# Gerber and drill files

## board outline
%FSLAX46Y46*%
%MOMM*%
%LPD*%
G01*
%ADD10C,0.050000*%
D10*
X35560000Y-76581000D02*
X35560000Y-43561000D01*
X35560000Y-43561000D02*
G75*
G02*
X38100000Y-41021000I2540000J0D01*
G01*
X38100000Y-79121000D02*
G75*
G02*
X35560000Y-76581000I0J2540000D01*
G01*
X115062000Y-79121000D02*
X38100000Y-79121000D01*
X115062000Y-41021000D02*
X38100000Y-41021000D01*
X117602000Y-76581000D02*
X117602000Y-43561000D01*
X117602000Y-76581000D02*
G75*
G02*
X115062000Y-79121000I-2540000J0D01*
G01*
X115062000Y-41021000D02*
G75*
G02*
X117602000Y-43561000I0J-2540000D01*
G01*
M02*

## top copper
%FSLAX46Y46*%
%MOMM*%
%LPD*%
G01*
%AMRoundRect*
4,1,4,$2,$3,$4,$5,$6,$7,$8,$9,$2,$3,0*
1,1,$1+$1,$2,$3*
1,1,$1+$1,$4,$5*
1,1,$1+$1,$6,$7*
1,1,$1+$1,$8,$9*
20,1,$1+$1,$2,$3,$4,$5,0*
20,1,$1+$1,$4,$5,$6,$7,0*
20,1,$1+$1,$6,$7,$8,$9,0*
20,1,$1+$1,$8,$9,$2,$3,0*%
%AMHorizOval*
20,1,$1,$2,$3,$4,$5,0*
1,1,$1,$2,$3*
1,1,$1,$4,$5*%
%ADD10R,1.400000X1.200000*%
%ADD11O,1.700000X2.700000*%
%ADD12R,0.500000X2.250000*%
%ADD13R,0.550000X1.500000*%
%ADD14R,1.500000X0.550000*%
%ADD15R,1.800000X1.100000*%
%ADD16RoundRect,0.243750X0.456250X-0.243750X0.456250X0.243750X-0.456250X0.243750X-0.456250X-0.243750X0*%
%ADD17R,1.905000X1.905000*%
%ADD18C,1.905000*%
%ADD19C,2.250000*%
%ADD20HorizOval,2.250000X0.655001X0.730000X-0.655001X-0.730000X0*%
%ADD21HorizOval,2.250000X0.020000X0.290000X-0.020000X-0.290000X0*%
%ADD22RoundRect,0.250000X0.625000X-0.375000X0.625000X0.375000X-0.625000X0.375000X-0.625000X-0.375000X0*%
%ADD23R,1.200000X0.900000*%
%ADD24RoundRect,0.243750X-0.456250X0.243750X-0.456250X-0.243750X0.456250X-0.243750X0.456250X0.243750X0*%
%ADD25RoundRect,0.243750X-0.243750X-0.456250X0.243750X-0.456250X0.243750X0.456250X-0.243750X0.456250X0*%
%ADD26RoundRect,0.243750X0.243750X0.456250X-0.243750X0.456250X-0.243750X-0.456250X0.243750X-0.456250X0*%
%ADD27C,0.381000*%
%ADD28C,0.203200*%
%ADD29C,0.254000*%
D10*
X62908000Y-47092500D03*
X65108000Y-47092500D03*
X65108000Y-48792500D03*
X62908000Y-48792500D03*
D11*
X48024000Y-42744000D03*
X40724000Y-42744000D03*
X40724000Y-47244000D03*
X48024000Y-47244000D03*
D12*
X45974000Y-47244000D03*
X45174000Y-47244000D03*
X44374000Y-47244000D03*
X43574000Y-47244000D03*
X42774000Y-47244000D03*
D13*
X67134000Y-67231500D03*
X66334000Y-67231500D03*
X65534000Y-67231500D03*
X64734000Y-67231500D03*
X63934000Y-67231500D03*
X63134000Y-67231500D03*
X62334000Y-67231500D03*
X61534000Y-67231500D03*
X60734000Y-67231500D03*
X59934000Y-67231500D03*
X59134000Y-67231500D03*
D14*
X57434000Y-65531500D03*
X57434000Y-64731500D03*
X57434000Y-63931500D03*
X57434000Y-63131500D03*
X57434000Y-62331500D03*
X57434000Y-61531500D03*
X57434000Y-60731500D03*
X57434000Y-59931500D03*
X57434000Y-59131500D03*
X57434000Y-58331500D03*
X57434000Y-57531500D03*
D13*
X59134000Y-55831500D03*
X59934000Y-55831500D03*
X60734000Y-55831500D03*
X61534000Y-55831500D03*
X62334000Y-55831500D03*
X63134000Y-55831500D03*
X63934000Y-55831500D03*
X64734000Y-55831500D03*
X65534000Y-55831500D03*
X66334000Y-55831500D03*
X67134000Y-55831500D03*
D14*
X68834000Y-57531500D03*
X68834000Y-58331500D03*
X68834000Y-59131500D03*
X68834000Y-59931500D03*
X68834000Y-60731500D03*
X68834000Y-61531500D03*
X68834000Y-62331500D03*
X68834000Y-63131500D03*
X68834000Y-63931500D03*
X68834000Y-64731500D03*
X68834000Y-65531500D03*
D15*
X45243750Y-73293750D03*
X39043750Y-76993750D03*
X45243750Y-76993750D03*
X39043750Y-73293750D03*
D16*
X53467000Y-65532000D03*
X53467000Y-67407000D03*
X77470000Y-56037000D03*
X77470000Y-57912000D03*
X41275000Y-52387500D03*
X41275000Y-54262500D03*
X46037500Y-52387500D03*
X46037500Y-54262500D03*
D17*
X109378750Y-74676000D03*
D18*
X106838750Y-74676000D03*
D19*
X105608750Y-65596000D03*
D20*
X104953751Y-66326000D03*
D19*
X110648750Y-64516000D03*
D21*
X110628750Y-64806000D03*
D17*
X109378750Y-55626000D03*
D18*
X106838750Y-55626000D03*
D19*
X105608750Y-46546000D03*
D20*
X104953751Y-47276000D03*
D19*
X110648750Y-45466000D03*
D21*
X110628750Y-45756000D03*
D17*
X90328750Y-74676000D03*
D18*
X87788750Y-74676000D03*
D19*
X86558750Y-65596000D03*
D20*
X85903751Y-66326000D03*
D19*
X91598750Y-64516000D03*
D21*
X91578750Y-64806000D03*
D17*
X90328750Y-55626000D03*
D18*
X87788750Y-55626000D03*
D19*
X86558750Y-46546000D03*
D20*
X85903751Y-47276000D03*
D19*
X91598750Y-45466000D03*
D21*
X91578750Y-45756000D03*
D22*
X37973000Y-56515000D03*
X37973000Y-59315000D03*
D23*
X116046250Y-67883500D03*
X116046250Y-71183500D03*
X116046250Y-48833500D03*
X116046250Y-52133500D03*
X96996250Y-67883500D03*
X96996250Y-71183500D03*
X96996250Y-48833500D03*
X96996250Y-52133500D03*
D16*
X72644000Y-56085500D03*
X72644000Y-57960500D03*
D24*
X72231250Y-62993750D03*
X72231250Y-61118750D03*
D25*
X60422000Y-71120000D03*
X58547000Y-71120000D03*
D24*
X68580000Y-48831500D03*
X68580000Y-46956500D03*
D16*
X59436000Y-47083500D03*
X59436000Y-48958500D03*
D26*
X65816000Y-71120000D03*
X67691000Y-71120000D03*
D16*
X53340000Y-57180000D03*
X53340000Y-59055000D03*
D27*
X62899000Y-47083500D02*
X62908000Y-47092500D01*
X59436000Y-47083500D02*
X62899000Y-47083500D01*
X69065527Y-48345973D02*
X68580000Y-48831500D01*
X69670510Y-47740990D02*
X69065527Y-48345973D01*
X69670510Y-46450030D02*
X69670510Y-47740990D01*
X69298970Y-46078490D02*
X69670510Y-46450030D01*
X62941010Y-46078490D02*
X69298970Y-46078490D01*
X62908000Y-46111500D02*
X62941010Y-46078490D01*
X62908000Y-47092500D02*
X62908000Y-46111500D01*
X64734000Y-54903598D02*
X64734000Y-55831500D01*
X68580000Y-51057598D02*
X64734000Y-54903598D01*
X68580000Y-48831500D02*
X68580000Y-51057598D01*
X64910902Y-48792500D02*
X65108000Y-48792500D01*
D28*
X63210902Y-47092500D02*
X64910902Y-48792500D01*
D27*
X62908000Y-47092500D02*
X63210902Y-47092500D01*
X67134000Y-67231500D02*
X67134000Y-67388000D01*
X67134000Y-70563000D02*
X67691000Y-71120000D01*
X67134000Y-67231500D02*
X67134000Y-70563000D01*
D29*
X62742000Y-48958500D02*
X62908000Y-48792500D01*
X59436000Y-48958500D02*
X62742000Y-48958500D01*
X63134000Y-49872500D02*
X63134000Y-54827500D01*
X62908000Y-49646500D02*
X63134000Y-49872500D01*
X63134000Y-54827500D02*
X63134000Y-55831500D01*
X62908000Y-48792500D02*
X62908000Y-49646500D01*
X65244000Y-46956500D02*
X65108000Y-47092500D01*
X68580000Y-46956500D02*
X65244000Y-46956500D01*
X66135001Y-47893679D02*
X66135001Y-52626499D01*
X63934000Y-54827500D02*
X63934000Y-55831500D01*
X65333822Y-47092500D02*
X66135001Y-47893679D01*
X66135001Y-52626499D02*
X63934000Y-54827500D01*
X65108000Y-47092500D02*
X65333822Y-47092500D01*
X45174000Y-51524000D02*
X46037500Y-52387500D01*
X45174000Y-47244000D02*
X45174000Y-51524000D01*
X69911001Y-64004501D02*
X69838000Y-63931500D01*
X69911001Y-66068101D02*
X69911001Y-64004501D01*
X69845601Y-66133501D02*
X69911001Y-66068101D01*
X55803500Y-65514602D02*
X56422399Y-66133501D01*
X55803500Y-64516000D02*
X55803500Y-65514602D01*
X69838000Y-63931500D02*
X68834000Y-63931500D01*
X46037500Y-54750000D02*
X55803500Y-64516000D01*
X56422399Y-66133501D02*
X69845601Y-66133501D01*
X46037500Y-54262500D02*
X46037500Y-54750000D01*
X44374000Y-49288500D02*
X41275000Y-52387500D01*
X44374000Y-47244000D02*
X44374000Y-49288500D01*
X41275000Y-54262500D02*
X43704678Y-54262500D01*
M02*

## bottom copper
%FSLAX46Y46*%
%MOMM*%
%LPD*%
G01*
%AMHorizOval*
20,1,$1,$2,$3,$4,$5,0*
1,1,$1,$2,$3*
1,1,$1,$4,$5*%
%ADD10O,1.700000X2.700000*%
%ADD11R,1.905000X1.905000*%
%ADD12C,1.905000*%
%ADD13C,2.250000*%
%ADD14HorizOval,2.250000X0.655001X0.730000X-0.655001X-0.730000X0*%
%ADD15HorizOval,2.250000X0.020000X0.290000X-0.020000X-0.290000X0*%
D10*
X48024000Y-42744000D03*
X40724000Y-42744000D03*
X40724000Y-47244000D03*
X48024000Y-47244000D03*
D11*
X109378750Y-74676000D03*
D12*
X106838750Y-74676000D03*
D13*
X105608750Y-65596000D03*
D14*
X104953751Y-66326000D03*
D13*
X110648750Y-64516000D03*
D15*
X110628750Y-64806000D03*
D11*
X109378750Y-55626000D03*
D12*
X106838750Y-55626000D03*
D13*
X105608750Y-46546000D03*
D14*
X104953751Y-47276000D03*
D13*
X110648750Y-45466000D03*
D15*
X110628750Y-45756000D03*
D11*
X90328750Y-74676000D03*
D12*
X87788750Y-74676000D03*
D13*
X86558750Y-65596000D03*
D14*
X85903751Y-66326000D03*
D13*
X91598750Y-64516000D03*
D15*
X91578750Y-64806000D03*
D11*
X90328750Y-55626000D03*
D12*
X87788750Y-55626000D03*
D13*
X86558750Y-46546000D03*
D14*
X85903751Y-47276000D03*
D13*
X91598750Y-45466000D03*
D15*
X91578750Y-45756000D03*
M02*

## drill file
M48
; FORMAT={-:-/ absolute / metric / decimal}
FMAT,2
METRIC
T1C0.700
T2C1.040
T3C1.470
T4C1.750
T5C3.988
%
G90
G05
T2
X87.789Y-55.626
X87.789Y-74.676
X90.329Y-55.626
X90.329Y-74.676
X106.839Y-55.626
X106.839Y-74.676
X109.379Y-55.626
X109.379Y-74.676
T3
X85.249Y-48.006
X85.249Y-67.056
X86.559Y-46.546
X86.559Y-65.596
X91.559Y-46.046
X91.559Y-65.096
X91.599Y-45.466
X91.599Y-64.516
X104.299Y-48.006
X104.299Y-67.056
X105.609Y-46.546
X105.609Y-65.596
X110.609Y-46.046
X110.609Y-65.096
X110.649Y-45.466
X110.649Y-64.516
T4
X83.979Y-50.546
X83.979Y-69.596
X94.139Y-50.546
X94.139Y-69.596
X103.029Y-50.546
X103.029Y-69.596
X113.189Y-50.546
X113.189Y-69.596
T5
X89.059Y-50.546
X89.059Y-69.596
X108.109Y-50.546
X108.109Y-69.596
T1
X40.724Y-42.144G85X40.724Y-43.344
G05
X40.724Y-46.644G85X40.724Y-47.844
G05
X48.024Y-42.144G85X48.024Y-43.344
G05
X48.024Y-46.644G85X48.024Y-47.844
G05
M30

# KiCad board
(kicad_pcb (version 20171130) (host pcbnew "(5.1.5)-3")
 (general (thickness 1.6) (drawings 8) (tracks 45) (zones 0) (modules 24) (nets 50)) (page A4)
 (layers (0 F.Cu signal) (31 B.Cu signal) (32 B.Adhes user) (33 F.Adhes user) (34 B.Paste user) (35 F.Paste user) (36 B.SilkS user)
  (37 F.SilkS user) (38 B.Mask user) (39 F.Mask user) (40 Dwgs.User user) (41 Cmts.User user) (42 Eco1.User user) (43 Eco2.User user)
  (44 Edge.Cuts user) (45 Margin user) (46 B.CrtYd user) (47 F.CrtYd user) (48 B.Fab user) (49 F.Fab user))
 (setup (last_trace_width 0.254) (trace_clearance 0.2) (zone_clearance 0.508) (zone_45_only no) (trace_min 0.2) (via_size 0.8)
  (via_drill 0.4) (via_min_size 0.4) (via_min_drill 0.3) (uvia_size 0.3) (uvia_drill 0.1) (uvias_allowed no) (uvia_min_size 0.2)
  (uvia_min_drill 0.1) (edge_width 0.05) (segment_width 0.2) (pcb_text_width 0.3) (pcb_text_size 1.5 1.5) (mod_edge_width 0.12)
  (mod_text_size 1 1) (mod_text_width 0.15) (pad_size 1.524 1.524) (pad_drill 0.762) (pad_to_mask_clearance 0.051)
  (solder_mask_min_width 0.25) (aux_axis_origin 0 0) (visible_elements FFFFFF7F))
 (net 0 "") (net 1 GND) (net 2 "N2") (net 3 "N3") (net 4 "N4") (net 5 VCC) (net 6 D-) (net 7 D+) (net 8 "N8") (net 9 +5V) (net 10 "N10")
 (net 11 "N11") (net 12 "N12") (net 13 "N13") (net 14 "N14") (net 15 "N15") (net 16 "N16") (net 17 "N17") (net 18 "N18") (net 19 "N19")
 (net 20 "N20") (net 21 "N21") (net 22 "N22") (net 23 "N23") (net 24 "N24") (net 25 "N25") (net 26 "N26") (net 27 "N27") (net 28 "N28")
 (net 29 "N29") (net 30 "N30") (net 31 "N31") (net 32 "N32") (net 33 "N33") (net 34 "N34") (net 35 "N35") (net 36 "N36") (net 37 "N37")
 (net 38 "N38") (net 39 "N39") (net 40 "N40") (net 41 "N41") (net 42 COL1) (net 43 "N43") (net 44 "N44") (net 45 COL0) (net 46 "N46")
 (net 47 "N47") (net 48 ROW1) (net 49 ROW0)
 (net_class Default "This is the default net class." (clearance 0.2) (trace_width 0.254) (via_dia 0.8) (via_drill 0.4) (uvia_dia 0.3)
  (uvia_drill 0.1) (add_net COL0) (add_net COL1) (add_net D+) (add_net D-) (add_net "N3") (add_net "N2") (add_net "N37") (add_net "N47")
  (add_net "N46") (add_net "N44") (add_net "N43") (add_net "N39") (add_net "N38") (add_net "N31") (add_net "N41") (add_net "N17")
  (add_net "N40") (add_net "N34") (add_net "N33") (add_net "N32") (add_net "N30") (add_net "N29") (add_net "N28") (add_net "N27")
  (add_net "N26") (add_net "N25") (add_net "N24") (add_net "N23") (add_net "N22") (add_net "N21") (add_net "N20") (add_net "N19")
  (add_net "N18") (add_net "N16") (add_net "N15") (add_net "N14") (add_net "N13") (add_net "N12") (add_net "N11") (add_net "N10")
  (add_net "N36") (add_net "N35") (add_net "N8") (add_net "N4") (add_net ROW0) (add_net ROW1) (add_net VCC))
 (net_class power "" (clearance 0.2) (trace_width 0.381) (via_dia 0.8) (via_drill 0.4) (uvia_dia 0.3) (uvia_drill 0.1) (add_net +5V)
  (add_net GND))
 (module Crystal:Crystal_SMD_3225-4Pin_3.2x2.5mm (layer F.Cu) (at 64.008 47.9425)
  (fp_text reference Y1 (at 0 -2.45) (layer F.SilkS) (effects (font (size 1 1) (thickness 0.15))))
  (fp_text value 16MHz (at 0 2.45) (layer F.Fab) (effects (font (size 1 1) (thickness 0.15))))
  (pad 4 smd rect (at -1.1 -0.85) (size 1.4 1.2) (layers F.Cu F.Paste F.Mask) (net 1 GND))
  (pad 3 smd rect (at 1.1 -0.85) (size 1.4 1.2) (layers F.Cu F.Paste F.Mask) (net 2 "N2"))
  (pad 2 smd rect (at 1.1 0.85) (size 1.4 1.2) (layers F.Cu F.Paste F.Mask) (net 1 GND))
  (pad 1 smd rect (at -1.1 0.85) (size 1.4 1.2) (layers F.Cu F.Paste F.Mask) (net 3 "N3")))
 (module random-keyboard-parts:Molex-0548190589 (layer F.Cu) (at 44.374 42.744 270)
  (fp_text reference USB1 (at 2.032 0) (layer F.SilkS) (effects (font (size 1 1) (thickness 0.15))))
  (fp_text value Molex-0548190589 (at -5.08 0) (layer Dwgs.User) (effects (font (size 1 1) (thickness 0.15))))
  (pad 6 thru_hole oval (at 0 -3.65 270) (size 2.7 1.7) (drill oval 1.9 0.7) (layers *.Cu *.Mask) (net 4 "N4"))
  (pad 6 thru_hole oval (at 0 3.65 270) (size 2.7 1.7) (drill oval 1.9 0.7) (layers *.Cu *.Mask) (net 4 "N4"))
  (pad 6 thru_hole oval (at 4.5 3.65 270) (size 2.7 1.7) (drill oval 1.9 0.7) (layers *.Cu *.Mask) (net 4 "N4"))
  (pad 6 thru_hole oval (at 4.5 -3.65 270) (size 2.7 1.7) (drill oval 1.9 0.7) (layers *.Cu *.Mask) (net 4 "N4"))
  (pad 5 smd rect (at 4.5 -1.6 270) (size 2.25 0.5) (layers F.Cu F.Paste F.Mask) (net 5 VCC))
  (pad 4 smd rect (at 4.5 -0.8 270) (size 2.25 0.5) (layers F.Cu F.Paste F.Mask) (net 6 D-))
  (pad 3 smd rect (at 4.5 0 270) (size 2.25 0.5) (layers F.Cu F.Paste F.Mask) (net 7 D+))
  (pad 2 smd rect (at 4.5 0.8 270) (size 2.25 0.5) (layers F.Cu F.Paste F.Mask) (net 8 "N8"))
  (pad 1 smd rect (at 4.5 1.6 270) (size 2.25 0.5) (layers F.Cu F.Paste F.Mask) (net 1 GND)))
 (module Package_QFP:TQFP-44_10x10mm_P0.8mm (layer F.Cu) (at 63.134 61.5315 180)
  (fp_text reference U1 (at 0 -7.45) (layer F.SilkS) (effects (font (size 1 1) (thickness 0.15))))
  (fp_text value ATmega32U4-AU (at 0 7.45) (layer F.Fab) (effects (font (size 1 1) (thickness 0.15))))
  (pad 44 smd rect (at -4 -5.7 270) (size 1.5 0.55) (layers F.Cu F.Paste F.Mask) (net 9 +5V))
  (pad 43 smd rect (at -3.2 -5.7 270) (size 1.5 0.55) (layers F.Cu F.Paste F.Mask) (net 1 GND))
  (pad 42 smd rect (at -2.4 -5.7 270) (size 1.5 0.55) (layers F.Cu F.Paste F.Mask) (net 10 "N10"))
  (pad 41 smd rect (at -1.6 -5.7 270) (size 1.5 0.55) (layers F.Cu F.Paste F.Mask) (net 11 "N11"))
  (pad 40 smd rect (at -0.8 -5.7 270) (size 1.5 0.55) (layers F.Cu F.Paste F.Mask) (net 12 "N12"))
  (pad 39 smd rect (at 0 -5.7 270) (size 1.5 0.55) (layers F.Cu F.Paste F.Mask) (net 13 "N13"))
  (pad 38 smd rect (at 0.8 -5.7 270) (size 1.5 0.55) (layers F.Cu F.Paste F.Mask) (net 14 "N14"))
  (pad 37 smd rect (at 1.6 -5.7 270) (size 1.5 0.55) (layers F.Cu F.Paste F.Mask) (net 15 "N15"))
  (pad 36 smd rect (at 2.4 -5.7 270) (size 1.5 0.55) (layers F.Cu F.Paste F.Mask) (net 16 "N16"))
  (pad 35 smd rect (at 3.2 -5.7 270) (size 1.5 0.55) (layers F.Cu F.Paste F.Mask) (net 1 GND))
  (pad 34 smd rect (at 4 -5.7 270) (size 1.5 0.55) (layers F.Cu F.Paste F.Mask) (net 9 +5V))
  (pad 33 smd rect (at 5.7 -4 180) (size 1.5 0.55) (layers F.Cu F.Paste F.Mask) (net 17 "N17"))
  (pad 32 smd rect (at 5.7 -3.2 180) (size 1.5 0.55) (layers F.Cu F.Paste F.Mask) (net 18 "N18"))
  (pad 31 smd rect (at 5.7 -2.4 180) (size 1.5 0.55) (layers F.Cu F.Paste F.Mask) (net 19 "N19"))
  (pad 30 smd rect (at 5.7 -1.6 180) (size 1.5 0.55) (layers F.Cu F.Paste F.Mask) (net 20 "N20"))
  (pad 29 smd rect (at 5.7 -0.8 180) (size 1.5 0.55) (layers F.Cu F.Paste F.Mask) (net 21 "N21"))
  (pad 28 smd rect (at 5.7 0 180) (size 1.5 0.55) (layers F.Cu F.Paste F.Mask) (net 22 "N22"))
  (pad 27 smd rect (at 5.7 0.8 180) (size 1.5 0.55) (layers F.Cu F.Paste F.Mask) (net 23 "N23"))
  (pad 26 smd rect (at 5.7 1.6 180) (size 1.5 0.55) (layers F.Cu F.Paste F.Mask) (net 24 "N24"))
  (pad 25 smd rect (at 5.7 2.4 180) (size 1.5 0.55) (layers F.Cu F.Paste F.Mask) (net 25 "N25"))
  (pad 24 smd rect (at 5.7 3.2 180) (size 1.5 0.55) (layers F.Cu F.Paste F.Mask) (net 9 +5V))
  (pad 23 smd rect (at 5.7 4 180) (size 1.5 0.55) (layers F.Cu F.Paste F.Mask) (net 1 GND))
  (pad 22 smd rect (at 4 5.7 270) (size 1.5 0.55) (layers F.Cu F.Paste F.Mask) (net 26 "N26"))
  (pad 21 smd rect (at 3.2 5.7 270) (size 1.5 0.55) (layers F.Cu F.Paste F.Mask) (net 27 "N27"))
  (pad 20 smd rect (at 2.4 5.7 270) (size 1.5 0.55) (layers F.Cu F.Paste F.Mask) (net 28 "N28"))
  (pad 19 smd rect (at 1.6 5.7 270) (size 1.5 0.55) (layers F.Cu F.Paste F.Mask) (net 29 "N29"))
  (pad 18 smd rect (at 0.8 5.7 270) (size 1.5 0.55) (layers F.Cu F.Paste F.Mask) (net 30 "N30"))
  (pad 17 smd rect (at 0 5.7 270) (size 1.5 0.55) (layers F.Cu F.Paste F.Mask) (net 3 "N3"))
  (pad 16 smd rect (at -0.8 5.7 270) (size 1.5 0.55) (layers F.Cu F.Paste F.Mask) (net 2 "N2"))
  (pad 15 smd rect (at -1.6 5.7 270) (size 1.5 0.55) (layers F.Cu F.Paste F.Mask) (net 1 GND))
  (pad 14 smd rect (at -2.4 5.7 270) (size 1.5 0.55) (layers F.Cu F.Paste F.Mask) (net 9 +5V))
  (pad 13 smd rect (at -3.2 5.7 270) (size 1.5 0.55) (layers F.Cu F.Paste F.Mask) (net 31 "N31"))
  (pad 12 smd rect (at -4 5.7 270) (size 1.5 0.55) (layers F.Cu F.Paste F.Mask) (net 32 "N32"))
  (pad 11 smd rect (at -5.7 4 180) (size 1.5 0.55) (layers F.Cu F.Paste F.Mask) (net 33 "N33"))
  (pad 10 smd rect (at -5.7 3.2 180) (size 1.5 0.55) (layers F.Cu F.Paste F.Mask) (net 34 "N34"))
  (pad 9 smd rect (at -5.7 2.4 180) (size 1.5 0.55) (layers F.Cu F.Paste F.Mask) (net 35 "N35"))
  (pad 8 smd rect (at -5.7 1.6 180) (size 1.5 0.55) (layers F.Cu F.Paste F.Mask) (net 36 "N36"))
  (pad 7 smd rect (at -5.7 0.8 180) (size 1.5 0.55) (layers F.Cu F.Paste F.Mask) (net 9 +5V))
  (pad 6 smd rect (at -5.7 0 180) (size 1.5 0.55) (layers F.Cu F.Paste F.Mask) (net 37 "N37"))
  (pad 5 smd rect (at -5.7 -0.8 180) (size 1.5 0.55) (layers F.Cu F.Paste F.Mask) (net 1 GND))
  (pad 4 smd rect (at -5.7 -1.6 180) (size 1.5 0.55) (layers F.Cu F.Paste F.Mask) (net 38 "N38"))
  (pad 3 smd rect (at -5.7 -2.4 180) (size 1.5 0.55) (layers F.Cu F.Paste F.Mask) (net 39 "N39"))
  (pad 2 smd rect (at -5.7 -3.2 180) (size 1.5 0.55) (layers F.Cu F.Paste F.Mask) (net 9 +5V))
  (pad 1 smd rect (at -5.7 -4 180) (size 1.5 0.55) (layers F.Cu F.Paste F.Mask) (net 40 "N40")))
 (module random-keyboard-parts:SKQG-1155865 (layer F.Cu) (at 42.14375 75.14375 180)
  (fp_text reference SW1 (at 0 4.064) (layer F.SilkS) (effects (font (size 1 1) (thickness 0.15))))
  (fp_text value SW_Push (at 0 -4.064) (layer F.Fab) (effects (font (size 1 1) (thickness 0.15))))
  (pad 4 smd rect (at -3.1 1.85 180) (size 1.8 1.1) (layers F.Cu F.Paste F.Mask))
  (pad 3 smd rect (at 3.1 -1.85 180) (size 1.8 1.1) (layers F.Cu F.Paste F.Mask))
  (pad 2 smd rect (at -3.1 -1.85 180) (size 1.8 1.1) (layers F.Cu F.Paste F.Mask) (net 31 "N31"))
  (pad 1 smd rect (at 3.1 1.85 180) (size 1.8 1.1) (layers F.Cu F.Paste F.Mask) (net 1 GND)))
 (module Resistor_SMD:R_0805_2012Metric (layer F.Cu) (at 53.467 66.4695 90)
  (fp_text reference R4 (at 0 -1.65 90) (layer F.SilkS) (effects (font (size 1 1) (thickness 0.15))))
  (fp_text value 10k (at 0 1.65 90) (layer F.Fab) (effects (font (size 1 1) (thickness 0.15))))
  (pad 2 smd roundrect (at 0.9375 0 90) (size 0.975 1.4) (layers F.Cu F.Paste F.Mask) (roundrect_rratio 0.25) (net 17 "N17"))
  (pad 1 smd roundrect (at -0.9375 0 90) (size 0.975 1.4) (layers F.Cu F.Paste F.Mask) (roundrect_rratio 0.25) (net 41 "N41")))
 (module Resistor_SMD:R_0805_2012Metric (layer F.Cu) (at 77.47 56.9745 90)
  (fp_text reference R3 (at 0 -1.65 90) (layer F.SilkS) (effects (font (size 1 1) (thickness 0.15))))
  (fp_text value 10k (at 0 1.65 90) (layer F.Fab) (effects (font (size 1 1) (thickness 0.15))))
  (pad 2 smd roundrect (at 0.9375 0 90) (size 0.975 1.4) (layers F.Cu F.Paste F.Mask) (roundrect_rratio 0.25) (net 31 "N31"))
  (pad 1 smd roundrect (at -0.9375 0 90) (size 0.975 1.4) (layers F.Cu F.Paste F.Mask) (roundrect_rratio 0.25) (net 9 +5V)))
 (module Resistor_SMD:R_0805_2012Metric (layer F.Cu) (at 41.275 53.325 90)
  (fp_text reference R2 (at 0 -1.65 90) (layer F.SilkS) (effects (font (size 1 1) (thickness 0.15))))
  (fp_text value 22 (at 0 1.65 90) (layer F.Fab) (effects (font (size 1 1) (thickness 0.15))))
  (pad 2 smd roundrect (at 0.9375 0 90) (size 0.975 1.4) (layers F.Cu F.Paste F.Mask) (roundrect_rratio 0.25) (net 7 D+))
  (pad 1 smd roundrect (at -0.9375 0 90) (size 0.975 1.4) (layers F.Cu F.Paste F.Mask) (roundrect_rratio 0.25) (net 38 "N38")))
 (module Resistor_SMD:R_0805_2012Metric (layer F.Cu) (at 46.0375 53.325 90)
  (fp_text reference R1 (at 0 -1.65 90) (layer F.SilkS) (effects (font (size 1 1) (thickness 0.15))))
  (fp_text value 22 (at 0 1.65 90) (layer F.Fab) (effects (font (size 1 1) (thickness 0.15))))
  (pad 2 smd roundrect (at 0.9375 0 90) (size 0.975 1.4) (layers F.Cu F.Paste F.Mask) (roundrect_rratio 0.25) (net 6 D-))
  (pad 1 smd roundrect (at -0.9375 0 90) (size 0.975 1.4) (layers F.Cu F.Paste F.Mask) (roundrect_rratio 0.25) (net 39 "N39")))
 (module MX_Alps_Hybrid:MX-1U (layer F.Cu) (at 108.10875 69.596)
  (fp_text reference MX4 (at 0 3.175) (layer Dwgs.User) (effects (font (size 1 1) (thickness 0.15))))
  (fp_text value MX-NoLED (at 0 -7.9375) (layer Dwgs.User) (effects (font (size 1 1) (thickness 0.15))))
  (pad "" np_thru_hole circle (at 5.08 0 48.0996) (size 1.75 1.75) (drill 1.75) (layers *.Cu *.Mask))
  (pad "" np_thru_hole circle (at -5.08 0 48.0996) (size 1.75 1.75) (drill 1.75) (layers *.Cu *.Mask))
  (pad 4 thru_hole rect (at 1.27 5.08) (size 1.905 1.905) (drill 1.04) (layers *.Cu B.Mask))
  (pad 3 thru_hole circle (at -1.27 5.08) (size 1.905 1.905) (drill 1.04) (layers *.Cu B.Mask))
  (pad 1 thru_hole circle (at -2.5 -4) (size 2.25 2.25) (drill 1.47) (layers *.Cu B.Mask) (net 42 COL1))
  (pad "" np_thru_hole circle (at 0 0) (size 3.9878 3.9878) (drill 3.9878) (layers *.Cu *.Mask))
  (pad 1 thru_hole oval (at -3.81 -2.54 48.0996) (size 4.211556 2.25) (drill 1.47 (offset 0.980778 0)) (layers *.Cu B.Mask) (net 42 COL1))
  (pad 2 thru_hole circle (at 2.54 -5.08) (size 2.25 2.25) (drill 1.47) (layers *.Cu B.Mask) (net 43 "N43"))
  (pad 2 thru_hole oval (at 2.5 -4.5 86.0548) (size 2.831378 2.25) (drill 1.47 (offset 0.290689 0)) (layers *.Cu B.Mask) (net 43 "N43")))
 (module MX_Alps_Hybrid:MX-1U (layer F.Cu) (at 108.10875 50.546)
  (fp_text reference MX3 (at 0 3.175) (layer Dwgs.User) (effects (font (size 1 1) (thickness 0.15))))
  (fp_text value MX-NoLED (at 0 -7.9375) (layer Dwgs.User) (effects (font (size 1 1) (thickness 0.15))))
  (pad "" np_thru_hole circle (at 5.08 0 48.0996) (size 1.75 1.75) (drill 1.75) (layers *.Cu *.Mask))
  (pad "" np_thru_hole circle (at -5.08 0 48.0996) (size 1.75 1.75) (drill 1.75) (layers *.Cu *.Mask))
  (pad 4 thru_hole rect (at 1.27 5.08) (size 1.905 1.905) (drill 1.04) (layers *.Cu B.Mask))
  (pad 3 thru_hole circle (at -1.27 5.08) (size 1.905 1.905) (drill 1.04) (layers *.Cu B.Mask))
  (pad 1 thru_hole circle (at -2.5 -4) (size 2.25 2.25) (drill 1.47) (layers *.Cu B.Mask) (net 42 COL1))
  (pad "" np_thru_hole circle (at 0 0) (size 3.9878 3.9878) (drill 3.9878) (layers *.Cu *.Mask))
  (pad 1 thru_hole oval (at -3.81 -2.54 48.0996) (size 4.211556 2.25) (drill 1.47 (offset 0.980778 0)) (layers *.Cu B.Mask) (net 42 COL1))
  (pad 2 thru_hole circle (at 2.54 -5.08) (size 2.25 2.25) (drill 1.47) (layers *.Cu B.Mask) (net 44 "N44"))
  (pad 2 thru_hole oval (at 2.5 -4.5 86.0548) (size 2.831378 2.25) (drill 1.47 (offset 0.290689 0)) (layers *.Cu B.Mask) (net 44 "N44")))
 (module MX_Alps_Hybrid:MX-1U (layer F.Cu) (at 89.05875 69.596)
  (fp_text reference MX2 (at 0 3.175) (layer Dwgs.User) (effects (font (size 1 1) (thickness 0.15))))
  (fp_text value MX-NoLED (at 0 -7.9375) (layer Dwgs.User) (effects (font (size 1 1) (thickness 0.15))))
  (pad "" np_thru_hole circle (at 5.08 0 48.0996) (size 1.75 1.75) (drill 1.75) (layers *.Cu *.Mask))
  (pad "" np_thru_hole circle (at -5.08 0 48.0996) (size 1.75 1.75) (drill 1.75) (layers *.Cu *.Mask))
  (pad 4 thru_hole rect (at 1.27 5.08) (size 1.905 1.905) (drill 1.04) (layers *.Cu B.Mask))
  (pad 3 thru_hole circle (at -1.27 5.08) (size 1.905 1.905) (drill 1.04) (layers *.Cu B.Mask))
  (pad 1 thru_hole circle (at -2.5 -4) (size 2.25 2.25) (drill 1.47) (layers *.Cu B.Mask) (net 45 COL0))
  (pad "" np_thru_hole circle (at 0 0) (size 3.9878 3.9878) (drill 3.9878) (layers *.Cu *.Mask))
  (pad 1 thru_hole oval (at -3.81 -2.54 48.0996) (size 4.211556 2.25) (drill 1.47 (offset 0.980778 0)) (layers *.Cu B.Mask) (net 45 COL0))
  (pad 2 thru_hole circle (at 2.54 -5.08) (size 2.25 2.25) (drill 1.47) (layers *.Cu B.Mask) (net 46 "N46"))
  (pad 2 thru_hole oval (at 2.5 -4.5 86.0548) (size 2.831378 2.25) (drill 1.47 (offset 0.290689 0)) (layers *.Cu B.Mask) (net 46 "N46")))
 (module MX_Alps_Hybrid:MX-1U (layer F.Cu) (at 89.05875 50.546)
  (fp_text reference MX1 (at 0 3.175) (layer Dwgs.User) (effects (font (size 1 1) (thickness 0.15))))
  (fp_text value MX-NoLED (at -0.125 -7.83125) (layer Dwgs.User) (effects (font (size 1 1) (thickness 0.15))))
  (pad "" np_thru_hole circle (at 5.08 0 48.0996) (size 1.75 1.75) (drill 1.75) (layers *.Cu *.Mask))
  (pad "" np_thru_hole circle (at -5.08 0 48.0996) (size 1.75 1.75) (drill 1.75) (layers *.Cu *.Mask))
  (pad 4 thru_hole rect (at 1.27 5.08) (size 1.905 1.905) (drill 1.04) (layers *.Cu B.Mask))
  (pad 3 thru_hole circle (at -1.27 5.08) (size 1.905 1.905) (drill 1.04) (layers *.Cu B.Mask))
  (pad 1 thru_hole circle (at -2.5 -4) (size 2.25 2.25) (drill 1.47) (layers *.Cu B.Mask) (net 45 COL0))
  (pad "" np_thru_hole circle (at 0 0) (size 3.9878 3.9878) (drill 3.9878) (layers *.Cu *.Mask))
  (pad 1 thru_hole oval (at -3.81 -2.54 48.0996) (size 4.211556 2.25) (drill 1.47 (offset 0.980778 0)) (layers *.Cu B.Mask) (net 45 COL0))
  (pad 2 thru_hole circle (at 2.54 -5.08) (size 2.25 2.25) (drill 1.47) (layers *.Cu B.Mask) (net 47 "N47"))
  (pad 2 thru_hole oval (at 2.5 -4.5 86.0548) (size 2.831378 2.25) (drill 1.47 (offset 0.290689 0)) (layers *.Cu B.Mask) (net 47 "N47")))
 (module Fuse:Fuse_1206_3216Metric (layer F.Cu) (at 37.973 57.915 90)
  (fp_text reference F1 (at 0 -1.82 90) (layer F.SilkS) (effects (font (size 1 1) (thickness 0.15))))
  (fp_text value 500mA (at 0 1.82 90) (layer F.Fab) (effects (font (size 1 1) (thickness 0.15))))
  (pad 2 smd roundrect (at 1.4 0 90) (size 1.25 1.75) (layers F.Cu F.Paste F.Mask) (roundrect_rratio 0.2) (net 5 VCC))
  (pad 1 smd roundrect (at -1.4 0 90) (size 1.25 1.75) (layers F.Cu F.Paste F.Mask) (roundrect_rratio 0.2) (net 9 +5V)))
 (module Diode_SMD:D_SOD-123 (layer F.Cu) (at 116.04625 69.5335 90)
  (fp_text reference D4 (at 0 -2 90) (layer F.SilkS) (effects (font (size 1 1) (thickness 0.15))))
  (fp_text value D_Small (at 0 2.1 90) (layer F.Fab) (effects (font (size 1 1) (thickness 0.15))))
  (pad 2 smd rect (at 1.65 0 90) (size 0.9 1.2) (layers F.Cu F.Paste F.Mask) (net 43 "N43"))
  (pad 1 smd rect (at -1.65 0 90) (size 0.9 1.2) (layers F.Cu F.Paste F.Mask) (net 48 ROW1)))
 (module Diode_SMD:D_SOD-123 (layer F.Cu) (at 116.04625 50.4835 90)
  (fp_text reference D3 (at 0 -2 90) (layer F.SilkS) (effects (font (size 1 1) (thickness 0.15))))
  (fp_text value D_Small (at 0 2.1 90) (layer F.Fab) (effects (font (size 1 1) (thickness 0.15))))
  (pad 2 smd rect (at 1.65 0 90) (size 0.9 1.2) (layers F.Cu F.Paste F.Mask) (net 44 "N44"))
  (pad 1 smd rect (at -1.65 0 90) (size 0.9 1.2) (layers F.Cu F.Paste F.Mask) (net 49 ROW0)))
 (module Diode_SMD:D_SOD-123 (layer F.Cu) (at 96.99625 69.5335 90)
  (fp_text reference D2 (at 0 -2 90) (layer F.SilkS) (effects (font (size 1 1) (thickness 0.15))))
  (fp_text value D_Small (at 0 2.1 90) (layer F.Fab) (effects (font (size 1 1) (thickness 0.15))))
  (pad 2 smd rect (at 1.65 0 90) (size 0.9 1.2) (layers F.Cu F.Paste F.Mask) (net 46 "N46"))
  (pad 1 smd rect (at -1.65 0 90) (size 0.9 1.2) (layers F.Cu F.Paste F.Mask) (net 48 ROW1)))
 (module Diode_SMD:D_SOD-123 (layer F.Cu) (at 96.99625 50.4835 90)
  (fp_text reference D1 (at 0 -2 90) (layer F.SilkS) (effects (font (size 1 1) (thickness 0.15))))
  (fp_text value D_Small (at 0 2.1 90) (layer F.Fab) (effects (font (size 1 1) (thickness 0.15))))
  (pad 2 smd rect (at 1.65 0 90) (size 0.9 1.2) (layers F.Cu F.Paste F.Mask) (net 47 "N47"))
  (pad 1 smd rect (at -1.65 0 90) (size 0.9 1.2) (layers F.Cu F.Paste F.Mask) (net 49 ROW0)))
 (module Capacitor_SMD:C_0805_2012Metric (layer F.Cu) (at 72.644 57.023 90)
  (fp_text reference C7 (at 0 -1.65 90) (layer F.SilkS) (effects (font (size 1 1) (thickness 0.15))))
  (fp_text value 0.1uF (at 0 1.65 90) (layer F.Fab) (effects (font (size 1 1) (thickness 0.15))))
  (pad 2 smd roundrect (at 0.9375 0 90) (size 0.975 1.4) (layers F.Cu F.Paste F.Mask) (roundrect_rratio 0.25) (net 1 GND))
  (pad 1 smd roundrect (at -0.9375 0 90) (size 0.975 1.4) (layers F.Cu F.Paste F.Mask) (roundrect_rratio 0.25) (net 9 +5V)))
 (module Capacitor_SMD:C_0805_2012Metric (layer F.Cu) (at 72.23125 62.05625 270)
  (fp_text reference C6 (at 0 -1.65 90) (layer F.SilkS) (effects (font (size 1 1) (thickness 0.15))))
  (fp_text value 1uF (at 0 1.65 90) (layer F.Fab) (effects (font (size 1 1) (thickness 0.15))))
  (pad 2 smd roundrect (at 0.9375 0 270) (size 0.975 1.4) (layers F.Cu F.Paste F.Mask) (roundrect_rratio 0.25) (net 1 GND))
  (pad 1 smd roundrect (at -0.9375 0 270) (size 0.975 1.4) (layers F.Cu F.Paste F.Mask) (roundrect_rratio 0.25) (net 37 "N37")))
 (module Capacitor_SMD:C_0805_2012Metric (layer F.Cu) (at 59.4845 71.12)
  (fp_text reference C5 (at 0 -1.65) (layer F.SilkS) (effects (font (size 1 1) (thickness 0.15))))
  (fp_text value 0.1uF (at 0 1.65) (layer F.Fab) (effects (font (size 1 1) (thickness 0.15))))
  (pad 2 smd roundrect (at 0.9375 0) (size 0.975 1.4) (layers F.Cu F.Paste F.Mask) (roundrect_rratio 0.25) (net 1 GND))
  (pad 1 smd roundrect (at -0.9375 0) (size 0.975 1.4) (layers F.Cu F.Paste F.Mask) (roundrect_rratio 0.25) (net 9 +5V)))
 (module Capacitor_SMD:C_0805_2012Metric (layer F.Cu) (at 68.58 47.894 270)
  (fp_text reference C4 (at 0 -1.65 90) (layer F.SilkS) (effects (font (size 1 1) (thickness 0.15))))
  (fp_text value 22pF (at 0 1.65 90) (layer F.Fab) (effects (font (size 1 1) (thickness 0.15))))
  (pad 2 smd roundrect (at 0.9375 0 270) (size 0.975 1.4) (layers F.Cu F.Paste F.Mask) (roundrect_rratio 0.25) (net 1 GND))
  (pad 1 smd roundrect (at -0.9375 0 270) (size 0.975 1.4) (layers F.Cu F.Paste F.Mask) (roundrect_rratio 0.25) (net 2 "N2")))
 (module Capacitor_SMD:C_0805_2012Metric (layer F.Cu) (at 59.436 48.021 90)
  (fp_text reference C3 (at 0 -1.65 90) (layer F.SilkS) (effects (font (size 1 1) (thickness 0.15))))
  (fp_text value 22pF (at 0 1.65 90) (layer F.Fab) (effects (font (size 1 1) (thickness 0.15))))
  (pad 2 smd roundrect (at 0.9375 0 90) (size 0.975 1.4) (layers F.Cu F.Paste F.Mask) (roundrect_rratio 0.25) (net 1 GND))
  (pad 1 smd roundrect (at -0.9375 0 90) (size 0.975 1.4) (layers F.Cu F.Paste F.Mask) (roundrect_rratio 0.25) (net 3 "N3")))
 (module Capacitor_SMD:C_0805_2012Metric (layer F.Cu) (at 66.7535 71.12 180)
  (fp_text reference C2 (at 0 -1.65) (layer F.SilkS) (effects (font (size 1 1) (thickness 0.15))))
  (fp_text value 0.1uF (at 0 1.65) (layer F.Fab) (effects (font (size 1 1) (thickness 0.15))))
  (pad 2 smd roundrect (at 0.9375 0 180) (size 0.975 1.4) (layers F.Cu F.Paste F.Mask) (roundrect_rratio 0.25) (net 1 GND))
  (pad 1 smd roundrect (at -0.9375 0 180) (size 0.975 1.4) (layers F.Cu F.Paste F.Mask) (roundrect_rratio 0.25) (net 9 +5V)))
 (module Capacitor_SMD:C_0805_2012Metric (layer F.Cu) (at 53.34 58.1175 90)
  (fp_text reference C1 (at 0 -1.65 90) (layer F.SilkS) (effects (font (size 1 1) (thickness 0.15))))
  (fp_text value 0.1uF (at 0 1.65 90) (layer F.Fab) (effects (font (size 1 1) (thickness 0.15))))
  (pad 2 smd roundrect (at 0.9375 0 90) (size 0.975 1.4) (layers F.Cu F.Paste F.Mask) (roundrect_rratio 0.25) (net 1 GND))
  (pad 1 smd roundrect (at -0.9375 0 90) (size 0.975 1.4) (layers F.Cu F.Paste F.Mask) (roundrect_rratio 0.25) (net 9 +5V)))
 (gr_line (start 35.56 76.581) (end 35.56 43.561) (layer Edge.Cuts) (width 0.05))
 (gr_arc (start 38.1 43.561) (end 38.1 41.021) (angle -90) (layer Edge.Cuts) (width 0.05))
 (gr_arc (start 38.1 76.581) (end 35.56 76.581) (angle -90) (layer Edge.Cuts) (width 0.05))
 (gr_line (start 115.062 79.121) (end 38.1 79.121) (layer Edge.Cuts) (width 0.05))
 (gr_line (start 115.062 41.021) (end 38.1 41.021) (layer Edge.Cuts) (width 0.05))
 (gr_line (start 117.602 76.581) (end 117.602 43.561) (layer Edge.Cuts) (width 0.05))
 (gr_arc (start 115.062 76.581) (end 115.062 79.121) (angle -90) (layer Edge.Cuts) (width 0.05))
 (gr_arc (start 115.062 43.561) (end 117.602 43.561) (angle -90) (layer Edge.Cuts) (width 0.05))
 (segment (start 62.899 47.0835) (end 62.908 47.0925) (width 0.381) (layer F.Cu) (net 1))
 (segment (start 59.436 47.0835) (end 62.899 47.0835) (width 0.381) (layer F.Cu) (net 1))
 (segment (start 69.065527 48.345973) (end 68.58 48.8315) (width 0.381) (layer F.Cu) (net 1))
 (segment (start 69.67051 47.74099) (end 69.065527 48.345973) (width 0.381) (layer F.Cu) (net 1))
 (segment (start 69.67051 46.45003) (end 69.67051 47.74099) (width 0.381) (layer F.Cu) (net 1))
 (segment (start 69.29897 46.07849) (end 69.67051 46.45003) (width 0.381) (layer F.Cu) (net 1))
 (segment (start 62.94101 46.07849) (end 69.29897 46.07849) (width 0.381) (layer F.Cu) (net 1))
 (segment (start 62.908 46.1115) (end 62.94101 46.07849) (width 0.381) (layer F.Cu) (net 1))
 (segment (start 62.908 47.0925) (end 62.908 46.1115) (width 0.381) (layer F.Cu) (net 1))
 (segment (start 64.734 54.903598) (end 64.734 55.8315) (width 0.381) (layer F.Cu) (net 1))
 (segment (start 68.58 51.057598) (end 64.734 54.903598) (width 0.381) (layer F.Cu) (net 1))
 (segment (start 68.58 48.8315) (end 68.58 51.057598) (width 0.381) (layer F.Cu) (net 1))
 (segment (start 64.910902 48.7925) (end 65.108 48.7925) (width 0.381) (layer F.Cu) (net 1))
 (segment (start 63.210902 47.0925) (end 64.910902 48.7925) (width 0.2032) (layer F.Cu) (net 1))
 (segment (start 62.908 47.0925) (end 63.210902 47.0925) (width 0.381) (layer F.Cu) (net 1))
 (segment (start 67.134 67.2315) (end 67.134 67.388) (width 0.381) (layer F.Cu) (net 9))
 (segment (start 67.134 70.563) (end 67.691 71.12) (width 0.381) (layer F.Cu) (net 9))
 (segment (start 67.134 67.2315) (end 67.134 70.563) (width 0.381) (layer F.Cu) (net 9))
 (segment (start 62.742 48.9585) (end 62.908 48.7925) (width 0.254) (layer F.Cu) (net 3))
 (segment (start 59.436 48.9585) (end 62.742 48.9585) (width 0.254) (layer F.Cu) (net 3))
 (segment (start 63.134 49.8725) (end 63.134 54.8275) (width 0.254) (layer F.Cu) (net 3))
 (segment (start 62.908 49.6465) (end 63.134 49.8725) (width 0.254) (layer F.Cu) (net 3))
 (segment (start 63.134 54.8275) (end 63.134 55.8315) (width 0.254) (layer F.Cu) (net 3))
 (segment (start 62.908 48.7925) (end 62.908 49.6465) (width 0.254) (layer F.Cu) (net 3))
 (segment (start 65.244 46.9565) (end 65.108 47.0925) (width 0.254) (layer F.Cu) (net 2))
 (segment (start 68.58 46.9565) (end 65.244 46.9565) (width 0.254) (layer F.Cu) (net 2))
 (segment (start 66.135001 47.893679) (end 66.135001 52.626499) (width 0.254) (layer F.Cu) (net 2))
 (segment (start 63.934 54.8275) (end 63.934 55.8315) (width 0.254) (layer F.Cu) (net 2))
 (segment (start 65.333822 47.0925) (end 66.135001 47.893679) (width 0.254) (layer F.Cu) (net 2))
 (segment (start 66.135001 52.626499) (end 63.934 54.8275) (width 0.254) (layer F.Cu) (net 2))
 (segment (start 65.108 47.0925) (end 65.333822 47.0925) (width 0.254) (layer F.Cu) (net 2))
 (segment (start 45.174 51.524) (end 46.0375 52.3875) (width 0.254) (layer F.Cu) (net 6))
 (segment (start 45.174 47.244) (end 45.174 51.524) (width 0.254) (layer F.Cu) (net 6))
 (segment (start 69.911001 64.004501) (end 69.838 63.9315) (width 0.254) (layer F.Cu) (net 39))
 (segment (start 69.911001 66.068101) (end 69.911001 64.004501) (width 0.254) (layer F.Cu) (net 39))
 (segment (start 69.845601 66.133501) (end 69.911001 66.068101) (width 0.254) (layer F.Cu) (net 39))
 (segment (start 55.8035 65.514602) (end 56.422399 66.133501) (width 0.254) (layer F.Cu) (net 39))
 (segment (start 55.8035 64.516) (end 55.8035 65.514602) (width 0.254) (layer F.Cu) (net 39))
 (segment (start 69.838 63.9315) (end 68.834 63.9315) (width 0.254) (layer F.Cu) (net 39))
 (segment (start 46.0375 54.75) (end 55.8035 64.516) (width 0.254) (layer F.Cu) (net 39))
 (segment (start 56.422399 66.133501) (end 69.845601 66.133501) (width 0.254) (layer F.Cu) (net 39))
 (segment (start 46.0375 54.2625) (end 46.0375 54.75) (width 0.254) (layer F.Cu) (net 39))
 (segment (start 44.374 49.2885) (end 41.275 52.3875) (width 0.254) (layer F.Cu) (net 7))
 (segment (start 44.374 47.244) (end 44.374 49.2885) (width 0.254) (layer F.Cu) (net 7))
 (segment (start 41.275 54.2625) (end 43.704678 54.2625) (width 0.254) (layer F.Cu) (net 38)))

